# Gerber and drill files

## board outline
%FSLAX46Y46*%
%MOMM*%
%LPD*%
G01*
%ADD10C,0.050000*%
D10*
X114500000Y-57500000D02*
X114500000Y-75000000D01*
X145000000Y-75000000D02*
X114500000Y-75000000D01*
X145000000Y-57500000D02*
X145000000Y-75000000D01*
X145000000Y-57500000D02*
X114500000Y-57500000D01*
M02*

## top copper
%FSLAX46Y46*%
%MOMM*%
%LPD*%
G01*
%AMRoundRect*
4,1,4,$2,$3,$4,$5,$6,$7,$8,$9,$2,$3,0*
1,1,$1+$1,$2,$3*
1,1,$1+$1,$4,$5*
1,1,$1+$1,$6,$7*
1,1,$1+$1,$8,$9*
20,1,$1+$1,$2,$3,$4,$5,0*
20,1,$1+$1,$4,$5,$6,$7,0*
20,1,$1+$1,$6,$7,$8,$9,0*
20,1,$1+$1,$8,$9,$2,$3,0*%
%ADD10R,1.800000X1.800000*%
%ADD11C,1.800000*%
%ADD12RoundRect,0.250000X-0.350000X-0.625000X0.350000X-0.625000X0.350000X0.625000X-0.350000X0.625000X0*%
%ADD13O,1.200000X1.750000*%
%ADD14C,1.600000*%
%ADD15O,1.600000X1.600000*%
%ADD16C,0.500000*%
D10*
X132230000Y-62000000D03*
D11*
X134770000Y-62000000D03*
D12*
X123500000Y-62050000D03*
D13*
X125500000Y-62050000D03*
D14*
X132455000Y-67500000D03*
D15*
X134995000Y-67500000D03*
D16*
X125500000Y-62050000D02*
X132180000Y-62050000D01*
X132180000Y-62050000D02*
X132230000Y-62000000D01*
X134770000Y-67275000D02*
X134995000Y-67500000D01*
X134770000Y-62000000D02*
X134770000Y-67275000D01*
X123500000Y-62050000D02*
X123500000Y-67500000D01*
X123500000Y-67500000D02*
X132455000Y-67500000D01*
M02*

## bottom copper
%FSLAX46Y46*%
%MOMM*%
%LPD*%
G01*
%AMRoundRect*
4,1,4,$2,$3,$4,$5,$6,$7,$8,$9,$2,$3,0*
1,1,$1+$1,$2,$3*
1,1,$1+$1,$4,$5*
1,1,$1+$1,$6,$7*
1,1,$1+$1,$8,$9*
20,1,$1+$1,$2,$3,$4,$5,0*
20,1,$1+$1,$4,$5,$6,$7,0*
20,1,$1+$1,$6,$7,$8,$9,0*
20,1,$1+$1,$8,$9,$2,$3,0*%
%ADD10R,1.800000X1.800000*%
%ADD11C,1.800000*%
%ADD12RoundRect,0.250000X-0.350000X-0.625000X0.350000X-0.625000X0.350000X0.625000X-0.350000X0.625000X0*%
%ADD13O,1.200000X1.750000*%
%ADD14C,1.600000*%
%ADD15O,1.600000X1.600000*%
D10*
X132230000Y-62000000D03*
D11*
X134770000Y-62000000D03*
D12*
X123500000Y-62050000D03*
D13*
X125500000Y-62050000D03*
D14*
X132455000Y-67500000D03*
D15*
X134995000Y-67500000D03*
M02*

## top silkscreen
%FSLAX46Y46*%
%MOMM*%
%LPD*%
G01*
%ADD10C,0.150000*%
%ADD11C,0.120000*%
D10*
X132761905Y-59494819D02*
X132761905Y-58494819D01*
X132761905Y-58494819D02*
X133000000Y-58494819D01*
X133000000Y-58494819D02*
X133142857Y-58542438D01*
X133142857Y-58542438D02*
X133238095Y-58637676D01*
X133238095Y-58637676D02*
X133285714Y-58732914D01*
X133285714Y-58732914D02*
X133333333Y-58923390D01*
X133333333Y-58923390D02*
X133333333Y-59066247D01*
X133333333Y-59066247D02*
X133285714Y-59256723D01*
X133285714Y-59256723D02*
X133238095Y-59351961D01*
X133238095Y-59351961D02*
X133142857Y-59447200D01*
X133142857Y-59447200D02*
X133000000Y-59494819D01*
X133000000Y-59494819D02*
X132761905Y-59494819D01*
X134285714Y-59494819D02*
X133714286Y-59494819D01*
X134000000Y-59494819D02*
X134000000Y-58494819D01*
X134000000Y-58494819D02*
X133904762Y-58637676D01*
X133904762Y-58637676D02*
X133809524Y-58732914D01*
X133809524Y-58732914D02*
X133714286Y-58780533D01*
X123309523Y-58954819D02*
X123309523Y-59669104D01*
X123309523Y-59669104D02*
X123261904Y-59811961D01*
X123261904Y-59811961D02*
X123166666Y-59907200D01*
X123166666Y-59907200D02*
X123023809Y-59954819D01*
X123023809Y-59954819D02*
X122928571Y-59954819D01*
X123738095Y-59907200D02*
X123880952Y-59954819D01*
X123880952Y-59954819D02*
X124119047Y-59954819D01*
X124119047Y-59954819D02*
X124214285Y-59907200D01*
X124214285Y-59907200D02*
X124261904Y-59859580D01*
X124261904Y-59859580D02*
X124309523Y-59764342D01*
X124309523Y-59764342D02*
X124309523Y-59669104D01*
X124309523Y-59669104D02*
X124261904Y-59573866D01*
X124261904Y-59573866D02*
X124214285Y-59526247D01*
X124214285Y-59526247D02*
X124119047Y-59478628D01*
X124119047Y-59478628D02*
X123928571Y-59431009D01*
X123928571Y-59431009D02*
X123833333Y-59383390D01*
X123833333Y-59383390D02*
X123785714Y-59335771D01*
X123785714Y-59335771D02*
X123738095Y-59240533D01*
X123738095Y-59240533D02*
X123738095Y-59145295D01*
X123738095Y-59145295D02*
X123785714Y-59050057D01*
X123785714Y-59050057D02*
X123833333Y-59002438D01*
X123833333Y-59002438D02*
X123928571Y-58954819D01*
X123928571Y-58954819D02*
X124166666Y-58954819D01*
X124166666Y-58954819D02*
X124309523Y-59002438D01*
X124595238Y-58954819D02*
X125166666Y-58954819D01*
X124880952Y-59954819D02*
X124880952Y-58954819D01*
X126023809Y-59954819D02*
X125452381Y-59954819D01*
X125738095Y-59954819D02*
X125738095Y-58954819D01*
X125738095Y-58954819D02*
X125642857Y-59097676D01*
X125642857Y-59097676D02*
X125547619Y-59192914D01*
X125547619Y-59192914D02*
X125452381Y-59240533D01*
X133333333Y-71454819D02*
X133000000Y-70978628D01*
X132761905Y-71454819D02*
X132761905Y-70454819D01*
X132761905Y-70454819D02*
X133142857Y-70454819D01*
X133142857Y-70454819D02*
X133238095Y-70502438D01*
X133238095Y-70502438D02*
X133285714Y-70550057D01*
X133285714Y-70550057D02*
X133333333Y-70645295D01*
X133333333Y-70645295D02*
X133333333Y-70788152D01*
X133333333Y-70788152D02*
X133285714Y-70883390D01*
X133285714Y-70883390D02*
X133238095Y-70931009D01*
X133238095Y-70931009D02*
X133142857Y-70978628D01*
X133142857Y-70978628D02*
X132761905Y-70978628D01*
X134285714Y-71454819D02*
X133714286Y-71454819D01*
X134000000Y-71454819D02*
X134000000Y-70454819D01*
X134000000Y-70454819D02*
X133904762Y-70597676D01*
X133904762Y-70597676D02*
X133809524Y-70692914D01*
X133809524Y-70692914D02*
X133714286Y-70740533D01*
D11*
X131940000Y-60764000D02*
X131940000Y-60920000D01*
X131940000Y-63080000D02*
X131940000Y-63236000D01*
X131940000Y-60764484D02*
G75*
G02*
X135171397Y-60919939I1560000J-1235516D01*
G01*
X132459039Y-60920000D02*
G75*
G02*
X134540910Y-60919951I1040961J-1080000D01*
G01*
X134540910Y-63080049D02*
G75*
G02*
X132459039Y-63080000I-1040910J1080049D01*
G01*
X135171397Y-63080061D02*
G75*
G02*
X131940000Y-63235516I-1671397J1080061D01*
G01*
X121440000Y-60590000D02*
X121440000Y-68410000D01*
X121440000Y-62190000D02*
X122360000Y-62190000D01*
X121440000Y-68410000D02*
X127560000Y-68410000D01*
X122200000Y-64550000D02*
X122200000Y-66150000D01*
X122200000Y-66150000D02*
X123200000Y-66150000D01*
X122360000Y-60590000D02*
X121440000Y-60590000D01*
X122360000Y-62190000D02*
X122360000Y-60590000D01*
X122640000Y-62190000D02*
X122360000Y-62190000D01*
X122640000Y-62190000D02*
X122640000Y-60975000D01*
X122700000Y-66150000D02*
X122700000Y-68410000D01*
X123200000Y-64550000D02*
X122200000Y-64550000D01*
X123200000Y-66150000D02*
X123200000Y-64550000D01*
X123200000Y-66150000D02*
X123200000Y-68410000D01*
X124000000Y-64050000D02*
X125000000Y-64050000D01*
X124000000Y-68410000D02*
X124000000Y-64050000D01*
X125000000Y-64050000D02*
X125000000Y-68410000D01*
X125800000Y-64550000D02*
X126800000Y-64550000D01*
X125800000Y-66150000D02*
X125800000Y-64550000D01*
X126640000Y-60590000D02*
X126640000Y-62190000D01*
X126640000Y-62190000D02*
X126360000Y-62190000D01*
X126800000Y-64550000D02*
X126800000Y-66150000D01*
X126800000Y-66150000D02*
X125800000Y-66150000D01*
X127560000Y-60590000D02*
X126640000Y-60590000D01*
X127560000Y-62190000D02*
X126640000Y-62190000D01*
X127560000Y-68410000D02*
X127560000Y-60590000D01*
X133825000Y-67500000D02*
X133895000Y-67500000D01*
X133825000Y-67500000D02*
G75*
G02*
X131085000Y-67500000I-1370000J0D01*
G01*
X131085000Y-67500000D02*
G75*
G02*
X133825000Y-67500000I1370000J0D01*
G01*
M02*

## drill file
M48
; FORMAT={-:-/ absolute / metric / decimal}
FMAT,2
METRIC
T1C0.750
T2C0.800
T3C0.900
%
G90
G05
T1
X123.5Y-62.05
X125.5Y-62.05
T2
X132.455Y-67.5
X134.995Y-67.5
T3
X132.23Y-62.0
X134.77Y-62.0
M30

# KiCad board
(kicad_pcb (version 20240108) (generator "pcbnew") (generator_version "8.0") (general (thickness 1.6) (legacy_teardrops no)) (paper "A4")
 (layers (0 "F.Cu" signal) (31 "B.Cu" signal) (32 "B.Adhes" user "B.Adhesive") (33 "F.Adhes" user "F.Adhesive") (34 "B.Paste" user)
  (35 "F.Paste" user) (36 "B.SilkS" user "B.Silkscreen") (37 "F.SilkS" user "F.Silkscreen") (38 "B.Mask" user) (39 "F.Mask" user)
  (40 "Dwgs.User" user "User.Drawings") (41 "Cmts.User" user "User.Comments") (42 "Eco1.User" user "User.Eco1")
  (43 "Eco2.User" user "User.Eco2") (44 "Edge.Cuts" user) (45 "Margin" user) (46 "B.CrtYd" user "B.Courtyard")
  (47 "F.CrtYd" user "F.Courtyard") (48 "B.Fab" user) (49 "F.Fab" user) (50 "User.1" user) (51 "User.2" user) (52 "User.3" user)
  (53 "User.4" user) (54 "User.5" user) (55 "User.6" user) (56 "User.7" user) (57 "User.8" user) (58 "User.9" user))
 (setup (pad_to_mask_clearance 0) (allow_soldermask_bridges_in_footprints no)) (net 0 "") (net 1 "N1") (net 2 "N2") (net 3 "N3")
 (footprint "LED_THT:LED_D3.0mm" (layer "F.Cu") (at 132.23 62)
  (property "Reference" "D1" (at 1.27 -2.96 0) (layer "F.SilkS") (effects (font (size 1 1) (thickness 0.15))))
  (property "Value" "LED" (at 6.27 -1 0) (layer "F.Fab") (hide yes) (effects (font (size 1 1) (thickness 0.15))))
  (fp_line (start -0.29 -1.236) (end -0.29 -1.08) (stroke (width 0.12) (type solid)) (layer "F.SilkS"))
  (fp_line (start -0.29 1.08) (end -0.29 1.236) (stroke (width 0.12) (type solid)) (layer "F.SilkS"))
  (fp_arc (start -0.29 -1.235516) (mid 1.365624 -1.987701) (end 2.941397 -1.080061) (stroke (width 0.12) (type solid)) (layer "F.SilkS"))
  (fp_arc (start 0.229039 -1.08) (mid 1.269965 -1.5) (end 2.31091 -1.080049) (stroke (width 0.12) (type solid)) (layer "F.SilkS"))
  (fp_arc (start 2.31091 1.080049) (mid 1.269965 1.5) (end 0.229039 1.08) (stroke (width 0.12) (type solid)) (layer "F.SilkS"))
  (fp_arc (start 2.941397 1.080061) (mid 1.365624 1.987701) (end -0.29 1.235516) (stroke (width 0.12) (type solid)) (layer "F.SilkS"))
  (pad "1" thru_hole rect (at 0 0) (size 1.8 1.8) (drill 0.9) (layers "*.Cu" "*.Mask") (remove_unused_layers no) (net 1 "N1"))
  (pad "2" thru_hole circle (at 2.54 0) (size 1.8 1.8) (drill 0.9) (layers "*.Cu" "*.Mask") (remove_unused_layers no) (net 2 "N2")))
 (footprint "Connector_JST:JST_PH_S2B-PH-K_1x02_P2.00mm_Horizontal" (layer "F.Cu") (at 123.5 62.05)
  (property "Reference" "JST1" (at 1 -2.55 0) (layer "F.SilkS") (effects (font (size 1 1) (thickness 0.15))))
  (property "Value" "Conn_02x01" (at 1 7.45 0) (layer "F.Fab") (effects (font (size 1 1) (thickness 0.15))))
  (fp_line (start -2.06 -1.46) (end -2.06 6.36) (stroke (width 0.12) (type solid)) (layer "F.SilkS"))
  (fp_line (start -2.06 0.14) (end -1.14 0.14) (stroke (width 0.12) (type solid)) (layer "F.SilkS"))
  (fp_line (start -2.06 6.36) (end 4.06 6.36) (stroke (width 0.12) (type solid)) (layer "F.SilkS"))
  (fp_line (start -1.3 2.5) (end -1.3 4.1) (stroke (width 0.12) (type solid)) (layer "F.SilkS"))
  (fp_line (start -1.3 4.1) (end -0.3 4.1) (stroke (width 0.12) (type solid)) (layer "F.SilkS"))
  (fp_line (start -1.14 -1.46) (end -2.06 -1.46) (stroke (width 0.12) (type solid)) (layer "F.SilkS"))
  (fp_line (start -1.14 0.14) (end -1.14 -1.46) (stroke (width 0.12) (type solid)) (layer "F.SilkS"))
  (fp_line (start -0.86 0.14) (end -1.14 0.14) (stroke (width 0.12) (type solid)) (layer "F.SilkS"))
  (fp_line (start -0.86 0.14) (end -0.86 -1.075) (stroke (width 0.12) (type solid)) (layer "F.SilkS"))
  (fp_line (start -0.8 4.1) (end -0.8 6.36) (stroke (width 0.12) (type solid)) (layer "F.SilkS"))
  (fp_line (start -0.3 2.5) (end -1.3 2.5) (stroke (width 0.12) (type solid)) (layer "F.SilkS"))
  (fp_line (start -0.3 4.1) (end -0.3 2.5) (stroke (width 0.12) (type solid)) (layer "F.SilkS"))
  (fp_line (start -0.3 4.1) (end -0.3 6.36) (stroke (width 0.12) (type solid)) (layer "F.SilkS"))
  (fp_line (start 0.5 2) (end 1.5 2) (stroke (width 0.12) (type solid)) (layer "F.SilkS"))
  (fp_line (start 0.5 6.36) (end 0.5 2) (stroke (width 0.12) (type solid)) (layer "F.SilkS"))
  (fp_line (start 1.5 2) (end 1.5 6.36) (stroke (width 0.12) (type solid)) (layer "F.SilkS"))
  (fp_line (start 2.3 2.5) (end 3.3 2.5) (stroke (width 0.12) (type solid)) (layer "F.SilkS"))
  (fp_line (start 2.3 4.1) (end 2.3 2.5) (stroke (width 0.12) (type solid)) (layer "F.SilkS"))
  (fp_line (start 3.14 -1.46) (end 3.14 0.14) (stroke (width 0.12) (type solid)) (layer "F.SilkS"))
  (fp_line (start 3.14 0.14) (end 2.86 0.14) (stroke (width 0.12) (type solid)) (layer "F.SilkS"))
  (fp_line (start 3.3 2.5) (end 3.3 4.1) (stroke (width 0.12) (type solid)) (layer "F.SilkS"))
  (fp_line (start 3.3 4.1) (end 2.3 4.1) (stroke (width 0.12) (type solid)) (layer "F.SilkS"))
  (fp_line (start 4.06 -1.46) (end 3.14 -1.46) (stroke (width 0.12) (type solid)) (layer "F.SilkS"))
  (fp_line (start 4.06 0.14) (end 3.14 0.14) (stroke (width 0.12) (type solid)) (layer "F.SilkS"))
  (fp_line (start 4.06 6.36) (end 4.06 -1.46) (stroke (width 0.12) (type solid)) (layer "F.SilkS"))
  (pad "1" thru_hole roundrect (at 0 0) (size 1.2 1.75) (drill 0.75) (layers "*.Cu" "*.Mask") (remove_unused_layers no)
   (roundrect_rratio 0.208333) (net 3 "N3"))
  (pad "2" thru_hole oval (at 2 0) (size 1.2 1.75) (drill 0.75) (layers "*.Cu" "*.Mask") (remove_unused_layers no) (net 1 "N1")))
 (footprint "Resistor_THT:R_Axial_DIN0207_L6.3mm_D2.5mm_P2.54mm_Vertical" (layer "F.Cu") (at 132.455 67.5)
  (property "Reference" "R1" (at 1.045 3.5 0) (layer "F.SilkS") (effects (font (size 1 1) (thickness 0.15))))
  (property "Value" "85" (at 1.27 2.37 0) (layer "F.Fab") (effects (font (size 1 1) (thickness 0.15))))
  (fp_line (start 1.37 0) (end 1.44 0) (stroke (width 0.12) (type solid)) (layer "F.SilkS"))
  (fp_circle (center 0 0) (end 1.37 0) (stroke (width 0.12) (type solid)) (fill none) (layer "F.SilkS"))
  (pad "1" thru_hole circle (at 0 0) (size 1.6 1.6) (drill 0.8) (layers "*.Cu" "*.Mask") (remove_unused_layers no) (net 3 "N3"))
  (pad "2" thru_hole oval (at 2.54 0) (size 1.6 1.6) (drill 0.8) (layers "*.Cu" "*.Mask") (remove_unused_layers no) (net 2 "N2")))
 (gr_line (start 114.5 57.5) (end 114.5 75) (stroke (width 0.05) (type default)) (layer "Edge.Cuts"))
 (gr_line (start 145 75) (end 114.5 75) (stroke (width 0.05) (type default)) (layer "Edge.Cuts"))
 (gr_line (start 145 57.5) (end 145 75) (stroke (width 0.05) (type default)) (layer "Edge.Cuts"))
 (gr_line (start 145 57.5) (end 114.5 57.5) (stroke (width 0.05) (type default)) (layer "Edge.Cuts"))
 (segment (start 125.5 62.05) (end 132.18 62.05) (width 0.5) (layer "F.Cu") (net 1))
 (segment (start 132.18 62.05) (end 132.23 62) (width 0.5) (layer "F.Cu") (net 1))
 (segment (start 134.77 67.275) (end 134.995 67.5) (width 0.5) (layer "F.Cu") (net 2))
 (segment (start 134.77 62) (end 134.77 67.275) (width 0.5) (layer "F.Cu") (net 2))
 (segment (start 123.5 62.05) (end 123.5 67.5) (width 0.5) (layer "F.Cu") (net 3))
 (segment (start 123.5 67.5) (end 132.455 67.5) (width 0.5) (layer "F.Cu") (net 3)))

